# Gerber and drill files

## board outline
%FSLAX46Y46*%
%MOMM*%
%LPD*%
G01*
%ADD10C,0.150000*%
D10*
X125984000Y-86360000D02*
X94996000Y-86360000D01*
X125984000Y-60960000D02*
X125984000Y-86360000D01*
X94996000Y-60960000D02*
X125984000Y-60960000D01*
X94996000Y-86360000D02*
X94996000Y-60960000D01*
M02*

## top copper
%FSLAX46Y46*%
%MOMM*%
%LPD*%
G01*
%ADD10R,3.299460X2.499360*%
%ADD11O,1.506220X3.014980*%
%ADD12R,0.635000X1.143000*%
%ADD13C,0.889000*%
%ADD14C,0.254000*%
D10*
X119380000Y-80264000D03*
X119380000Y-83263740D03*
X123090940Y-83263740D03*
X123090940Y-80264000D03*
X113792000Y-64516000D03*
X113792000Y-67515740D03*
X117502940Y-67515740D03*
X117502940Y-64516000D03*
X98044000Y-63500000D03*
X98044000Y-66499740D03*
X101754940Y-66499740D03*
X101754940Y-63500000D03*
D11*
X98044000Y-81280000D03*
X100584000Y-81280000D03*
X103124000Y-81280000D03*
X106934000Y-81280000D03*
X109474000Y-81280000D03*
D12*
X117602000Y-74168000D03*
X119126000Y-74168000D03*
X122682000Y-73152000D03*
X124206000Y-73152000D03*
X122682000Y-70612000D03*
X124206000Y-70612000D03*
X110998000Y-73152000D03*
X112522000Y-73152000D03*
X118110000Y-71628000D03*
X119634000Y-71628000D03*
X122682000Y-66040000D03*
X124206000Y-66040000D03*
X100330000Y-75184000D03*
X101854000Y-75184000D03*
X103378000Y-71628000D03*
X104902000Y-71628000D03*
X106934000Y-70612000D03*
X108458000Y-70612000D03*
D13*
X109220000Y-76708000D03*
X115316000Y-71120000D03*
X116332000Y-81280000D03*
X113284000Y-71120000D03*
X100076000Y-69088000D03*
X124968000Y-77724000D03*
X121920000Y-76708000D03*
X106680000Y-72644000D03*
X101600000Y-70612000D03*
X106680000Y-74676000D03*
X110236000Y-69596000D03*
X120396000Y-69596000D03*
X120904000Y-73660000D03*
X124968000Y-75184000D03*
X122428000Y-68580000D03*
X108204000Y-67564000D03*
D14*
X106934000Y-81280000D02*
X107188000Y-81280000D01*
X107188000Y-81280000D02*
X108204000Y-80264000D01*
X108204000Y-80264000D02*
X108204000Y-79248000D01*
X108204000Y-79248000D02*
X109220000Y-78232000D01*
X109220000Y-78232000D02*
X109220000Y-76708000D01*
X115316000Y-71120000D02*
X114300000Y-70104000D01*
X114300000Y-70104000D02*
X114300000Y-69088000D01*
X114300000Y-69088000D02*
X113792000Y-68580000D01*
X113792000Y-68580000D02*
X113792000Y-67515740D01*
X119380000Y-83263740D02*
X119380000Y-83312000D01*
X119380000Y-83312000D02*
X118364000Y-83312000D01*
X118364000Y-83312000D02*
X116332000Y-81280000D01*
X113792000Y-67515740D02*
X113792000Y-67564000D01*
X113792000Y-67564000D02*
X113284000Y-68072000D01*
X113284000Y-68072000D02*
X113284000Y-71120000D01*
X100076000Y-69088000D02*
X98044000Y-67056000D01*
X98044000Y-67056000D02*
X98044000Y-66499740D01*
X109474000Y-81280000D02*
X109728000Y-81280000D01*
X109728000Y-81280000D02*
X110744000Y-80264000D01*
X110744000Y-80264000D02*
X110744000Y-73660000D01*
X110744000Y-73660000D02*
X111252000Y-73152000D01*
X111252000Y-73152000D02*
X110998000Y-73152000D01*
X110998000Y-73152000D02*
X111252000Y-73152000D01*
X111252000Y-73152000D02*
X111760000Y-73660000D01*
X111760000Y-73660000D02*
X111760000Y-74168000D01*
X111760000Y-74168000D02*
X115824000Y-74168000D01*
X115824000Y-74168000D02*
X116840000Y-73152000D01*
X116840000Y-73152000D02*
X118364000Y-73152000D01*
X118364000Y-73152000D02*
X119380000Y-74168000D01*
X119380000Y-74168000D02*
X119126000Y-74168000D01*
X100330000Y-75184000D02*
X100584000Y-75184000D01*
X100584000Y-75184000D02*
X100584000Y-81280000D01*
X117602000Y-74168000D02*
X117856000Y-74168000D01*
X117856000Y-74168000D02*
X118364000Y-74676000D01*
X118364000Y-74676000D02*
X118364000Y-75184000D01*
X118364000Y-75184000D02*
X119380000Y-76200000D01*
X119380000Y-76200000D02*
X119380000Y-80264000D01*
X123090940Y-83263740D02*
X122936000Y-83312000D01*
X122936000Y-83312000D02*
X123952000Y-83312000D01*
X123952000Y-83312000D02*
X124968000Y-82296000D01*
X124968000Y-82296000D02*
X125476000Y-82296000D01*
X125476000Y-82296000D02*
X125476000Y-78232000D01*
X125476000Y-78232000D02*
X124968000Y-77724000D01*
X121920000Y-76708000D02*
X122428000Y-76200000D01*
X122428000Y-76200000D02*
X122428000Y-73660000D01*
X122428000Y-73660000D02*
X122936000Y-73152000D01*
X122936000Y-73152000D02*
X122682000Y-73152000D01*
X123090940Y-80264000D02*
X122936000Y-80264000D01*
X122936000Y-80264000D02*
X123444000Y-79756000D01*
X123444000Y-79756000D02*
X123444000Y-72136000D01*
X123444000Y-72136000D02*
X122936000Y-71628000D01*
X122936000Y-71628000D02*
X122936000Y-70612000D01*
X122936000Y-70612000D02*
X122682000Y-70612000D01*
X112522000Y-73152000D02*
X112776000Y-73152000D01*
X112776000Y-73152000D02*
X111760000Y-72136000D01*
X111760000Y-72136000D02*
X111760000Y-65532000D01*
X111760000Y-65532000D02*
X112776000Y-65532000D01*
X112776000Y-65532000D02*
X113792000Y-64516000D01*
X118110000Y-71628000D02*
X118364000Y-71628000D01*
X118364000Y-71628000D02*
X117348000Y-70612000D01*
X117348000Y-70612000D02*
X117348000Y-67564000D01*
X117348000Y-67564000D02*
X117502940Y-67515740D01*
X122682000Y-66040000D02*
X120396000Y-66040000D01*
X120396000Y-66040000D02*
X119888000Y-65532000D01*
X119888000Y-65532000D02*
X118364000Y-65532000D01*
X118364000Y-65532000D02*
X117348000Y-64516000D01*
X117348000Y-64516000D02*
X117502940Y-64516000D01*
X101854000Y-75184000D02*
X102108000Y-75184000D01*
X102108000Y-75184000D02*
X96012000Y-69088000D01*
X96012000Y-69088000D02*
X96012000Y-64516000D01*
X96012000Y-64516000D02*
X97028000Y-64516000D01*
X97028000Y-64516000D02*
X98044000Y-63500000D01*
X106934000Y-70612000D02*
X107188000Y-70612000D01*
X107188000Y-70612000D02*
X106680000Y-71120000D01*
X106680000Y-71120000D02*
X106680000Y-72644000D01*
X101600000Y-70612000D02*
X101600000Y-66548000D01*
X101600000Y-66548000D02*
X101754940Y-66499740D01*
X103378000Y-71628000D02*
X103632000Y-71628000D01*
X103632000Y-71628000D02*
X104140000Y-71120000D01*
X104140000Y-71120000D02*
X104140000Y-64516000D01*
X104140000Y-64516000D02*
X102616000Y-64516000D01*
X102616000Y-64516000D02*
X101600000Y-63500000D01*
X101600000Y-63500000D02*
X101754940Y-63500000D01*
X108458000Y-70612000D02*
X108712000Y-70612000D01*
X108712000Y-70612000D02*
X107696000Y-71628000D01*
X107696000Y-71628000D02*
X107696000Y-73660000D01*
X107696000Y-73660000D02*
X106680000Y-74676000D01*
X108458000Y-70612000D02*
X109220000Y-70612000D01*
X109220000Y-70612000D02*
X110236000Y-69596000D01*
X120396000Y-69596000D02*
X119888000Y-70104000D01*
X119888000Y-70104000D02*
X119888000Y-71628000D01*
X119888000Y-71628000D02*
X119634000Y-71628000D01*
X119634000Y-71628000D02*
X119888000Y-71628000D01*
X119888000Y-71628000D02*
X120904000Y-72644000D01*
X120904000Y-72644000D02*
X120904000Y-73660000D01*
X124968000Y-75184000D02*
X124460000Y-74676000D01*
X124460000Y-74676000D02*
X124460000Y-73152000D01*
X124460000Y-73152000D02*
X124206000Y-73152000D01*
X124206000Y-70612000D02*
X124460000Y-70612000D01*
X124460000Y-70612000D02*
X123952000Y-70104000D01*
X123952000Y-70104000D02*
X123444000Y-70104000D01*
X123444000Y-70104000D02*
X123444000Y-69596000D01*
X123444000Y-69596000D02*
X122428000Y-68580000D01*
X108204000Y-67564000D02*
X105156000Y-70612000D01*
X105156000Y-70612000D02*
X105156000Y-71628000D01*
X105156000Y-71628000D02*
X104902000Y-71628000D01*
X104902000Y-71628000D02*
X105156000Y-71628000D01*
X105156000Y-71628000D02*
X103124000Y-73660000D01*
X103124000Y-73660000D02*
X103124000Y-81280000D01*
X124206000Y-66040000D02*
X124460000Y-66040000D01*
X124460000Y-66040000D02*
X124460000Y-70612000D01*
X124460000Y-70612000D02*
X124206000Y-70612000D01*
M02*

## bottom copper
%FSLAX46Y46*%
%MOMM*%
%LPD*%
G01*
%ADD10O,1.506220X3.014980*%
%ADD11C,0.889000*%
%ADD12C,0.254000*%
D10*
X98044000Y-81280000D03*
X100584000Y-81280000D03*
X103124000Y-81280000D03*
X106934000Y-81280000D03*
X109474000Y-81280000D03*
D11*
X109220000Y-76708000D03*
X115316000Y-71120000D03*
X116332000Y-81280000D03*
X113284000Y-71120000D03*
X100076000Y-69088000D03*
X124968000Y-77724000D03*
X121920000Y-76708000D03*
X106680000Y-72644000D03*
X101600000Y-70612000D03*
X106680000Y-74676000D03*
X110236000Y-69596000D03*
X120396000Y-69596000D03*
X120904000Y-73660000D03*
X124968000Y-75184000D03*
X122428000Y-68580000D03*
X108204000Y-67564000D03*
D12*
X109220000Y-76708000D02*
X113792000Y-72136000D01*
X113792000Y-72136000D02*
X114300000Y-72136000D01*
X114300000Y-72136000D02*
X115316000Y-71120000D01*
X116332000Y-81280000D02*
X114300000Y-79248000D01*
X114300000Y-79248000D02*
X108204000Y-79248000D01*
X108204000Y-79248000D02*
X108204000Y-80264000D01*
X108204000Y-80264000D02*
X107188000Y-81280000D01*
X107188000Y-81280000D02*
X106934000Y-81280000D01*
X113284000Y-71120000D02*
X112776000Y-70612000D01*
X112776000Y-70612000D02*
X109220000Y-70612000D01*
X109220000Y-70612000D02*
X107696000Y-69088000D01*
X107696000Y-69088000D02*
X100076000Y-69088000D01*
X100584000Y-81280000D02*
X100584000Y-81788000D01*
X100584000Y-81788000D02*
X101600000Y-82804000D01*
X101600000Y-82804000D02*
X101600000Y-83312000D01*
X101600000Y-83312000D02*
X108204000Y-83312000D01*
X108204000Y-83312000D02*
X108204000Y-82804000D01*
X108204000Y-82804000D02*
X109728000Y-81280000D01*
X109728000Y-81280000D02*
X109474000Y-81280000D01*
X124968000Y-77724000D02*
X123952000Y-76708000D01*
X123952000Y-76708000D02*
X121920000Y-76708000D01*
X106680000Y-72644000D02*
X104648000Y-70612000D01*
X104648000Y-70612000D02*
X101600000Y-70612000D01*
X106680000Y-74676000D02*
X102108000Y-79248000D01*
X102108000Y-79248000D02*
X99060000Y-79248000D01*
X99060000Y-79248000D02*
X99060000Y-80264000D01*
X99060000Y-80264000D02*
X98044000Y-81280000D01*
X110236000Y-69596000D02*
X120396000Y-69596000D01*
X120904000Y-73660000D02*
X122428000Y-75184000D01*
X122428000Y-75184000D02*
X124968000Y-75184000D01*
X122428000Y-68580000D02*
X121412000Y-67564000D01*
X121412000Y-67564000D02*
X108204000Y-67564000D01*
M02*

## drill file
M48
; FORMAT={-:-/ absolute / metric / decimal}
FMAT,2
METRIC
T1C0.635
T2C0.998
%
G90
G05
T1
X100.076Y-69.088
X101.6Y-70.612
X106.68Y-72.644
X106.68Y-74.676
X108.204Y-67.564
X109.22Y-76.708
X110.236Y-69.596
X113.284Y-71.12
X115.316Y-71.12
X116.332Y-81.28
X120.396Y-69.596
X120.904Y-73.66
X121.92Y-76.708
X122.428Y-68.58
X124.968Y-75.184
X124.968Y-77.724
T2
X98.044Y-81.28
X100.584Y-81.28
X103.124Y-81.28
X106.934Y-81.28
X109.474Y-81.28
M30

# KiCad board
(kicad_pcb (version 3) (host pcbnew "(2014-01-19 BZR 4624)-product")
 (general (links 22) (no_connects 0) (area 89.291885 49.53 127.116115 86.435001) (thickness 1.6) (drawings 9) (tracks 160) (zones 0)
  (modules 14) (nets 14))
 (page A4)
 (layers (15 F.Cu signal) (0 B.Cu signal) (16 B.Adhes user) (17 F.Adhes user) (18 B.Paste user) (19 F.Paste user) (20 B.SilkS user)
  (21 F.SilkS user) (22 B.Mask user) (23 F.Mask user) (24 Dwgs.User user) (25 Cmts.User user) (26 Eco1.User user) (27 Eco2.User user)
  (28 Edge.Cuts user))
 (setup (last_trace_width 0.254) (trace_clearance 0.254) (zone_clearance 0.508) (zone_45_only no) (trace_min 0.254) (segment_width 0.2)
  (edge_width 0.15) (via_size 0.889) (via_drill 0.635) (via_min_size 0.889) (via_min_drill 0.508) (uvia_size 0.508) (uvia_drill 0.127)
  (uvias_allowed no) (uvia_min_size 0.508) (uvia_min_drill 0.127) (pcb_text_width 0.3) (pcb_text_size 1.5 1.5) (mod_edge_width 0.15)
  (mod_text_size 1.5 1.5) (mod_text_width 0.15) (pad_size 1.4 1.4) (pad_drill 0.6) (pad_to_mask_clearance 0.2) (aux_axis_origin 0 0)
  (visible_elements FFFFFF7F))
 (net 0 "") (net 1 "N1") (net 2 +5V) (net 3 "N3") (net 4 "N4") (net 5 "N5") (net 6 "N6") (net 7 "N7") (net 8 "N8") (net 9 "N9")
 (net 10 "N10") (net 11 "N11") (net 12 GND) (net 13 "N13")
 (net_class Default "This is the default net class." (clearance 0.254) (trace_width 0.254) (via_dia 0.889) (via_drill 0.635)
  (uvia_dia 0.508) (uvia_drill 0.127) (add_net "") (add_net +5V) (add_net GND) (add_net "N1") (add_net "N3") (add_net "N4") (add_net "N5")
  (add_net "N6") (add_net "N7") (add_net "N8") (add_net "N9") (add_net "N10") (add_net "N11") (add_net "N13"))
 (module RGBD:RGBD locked (layer F.Cu) (at 119.38 77.724)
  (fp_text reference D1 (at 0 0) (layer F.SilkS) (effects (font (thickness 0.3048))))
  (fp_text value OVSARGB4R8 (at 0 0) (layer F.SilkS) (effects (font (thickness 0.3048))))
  (pad 1 smd rect (at 0 2.54) (size 3.29946 2.49936) (layers F.Cu F.Paste F.Mask) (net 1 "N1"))
  (pad 2 smd rect (at 0 5.53974) (size 3.29946 2.49936) (layers F.Cu F.Paste F.Mask) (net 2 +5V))
  (pad 3 smd rect (at 3.71094 5.53974) (size 3.29946 2.49936) (layers F.Cu F.Paste F.Mask) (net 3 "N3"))
  (pad 4 smd rect (at 3.71094 2.54) (size 3.29946 2.49936) (layers F.Cu F.Paste F.Mask) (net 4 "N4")))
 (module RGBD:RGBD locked (layer F.Cu) (at 113.792 61.976)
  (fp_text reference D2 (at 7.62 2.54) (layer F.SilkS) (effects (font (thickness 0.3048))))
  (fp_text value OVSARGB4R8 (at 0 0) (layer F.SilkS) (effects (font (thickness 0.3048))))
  (pad 1 smd rect (at 0 2.54) (size 3.29946 2.49936) (layers F.Cu F.Paste F.Mask) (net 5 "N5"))
  (pad 2 smd rect (at 0 5.53974) (size 3.29946 2.49936) (layers F.Cu F.Paste F.Mask) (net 2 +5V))
  (pad 3 smd rect (at 3.71094 5.53974) (size 3.29946 2.49936) (layers F.Cu F.Paste F.Mask) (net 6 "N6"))
  (pad 4 smd rect (at 3.71094 2.54) (size 3.29946 2.49936) (layers F.Cu F.Paste F.Mask) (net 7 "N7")))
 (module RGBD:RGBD (layer F.Cu) (at 98.044 60.96)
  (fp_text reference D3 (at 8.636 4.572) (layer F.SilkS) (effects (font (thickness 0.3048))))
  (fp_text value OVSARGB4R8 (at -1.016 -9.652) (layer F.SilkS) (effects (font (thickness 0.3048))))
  (pad 1 smd rect (at 0 2.54) (size 3.29946 2.49936) (layers F.Cu F.Paste F.Mask) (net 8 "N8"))
  (pad 2 smd rect (at 0 5.53974) (size 3.29946 2.49936) (layers F.Cu F.Paste F.Mask) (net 2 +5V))
  (pad 3 smd rect (at 3.71094 5.53974) (size 3.29946 2.49936) (layers F.Cu F.Paste F.Mask) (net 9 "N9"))
  (pad 4 smd rect (at 3.71094 2.54) (size 3.29946 2.49936) (layers F.Cu F.Paste F.Mask) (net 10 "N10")))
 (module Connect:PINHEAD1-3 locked (layer F.Cu) (at 100.584 81.28)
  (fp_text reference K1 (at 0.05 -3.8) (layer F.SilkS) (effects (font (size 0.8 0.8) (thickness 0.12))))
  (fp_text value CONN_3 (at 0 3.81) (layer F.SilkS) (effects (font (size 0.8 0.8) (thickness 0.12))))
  (pad 1 thru_hole oval (at -2.54 0) (size 1.50622 3.01498) (drill 0.99822) (layers *.Cu *.Mask F.SilkS) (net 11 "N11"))
  (pad 2 thru_hole oval (at 0 0) (size 1.50622 3.01498) (drill 0.99822) (layers *.Cu *.Mask F.SilkS) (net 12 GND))
  (pad 3 thru_hole oval (at 2.54 0) (size 1.50622 3.01498) (drill 0.99822) (layers *.Cu *.Mask F.SilkS) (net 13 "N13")))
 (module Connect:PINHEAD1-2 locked (layer F.Cu) (at 108.204 81.28)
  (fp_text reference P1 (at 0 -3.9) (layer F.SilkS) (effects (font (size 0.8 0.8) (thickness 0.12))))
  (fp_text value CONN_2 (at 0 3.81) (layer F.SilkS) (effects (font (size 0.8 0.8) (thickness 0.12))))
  (pad 1 thru_hole oval (at -1.27 0) (size 1.50622 3.01498) (drill 0.99822) (layers *.Cu *.Mask F.SilkS) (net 2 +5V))
  (pad 2 thru_hole oval (at 1.27 0) (size 1.50622 3.01498) (drill 0.99822) (layers *.Cu *.Mask F.SilkS) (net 12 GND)))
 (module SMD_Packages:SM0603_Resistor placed (layer F.Cu) (at 118.364 74.168)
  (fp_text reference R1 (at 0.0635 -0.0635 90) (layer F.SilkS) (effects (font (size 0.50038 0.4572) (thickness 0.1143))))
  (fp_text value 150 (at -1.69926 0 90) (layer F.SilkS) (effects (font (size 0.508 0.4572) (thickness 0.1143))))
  (pad 1 smd rect (at -0.762 0) (size 0.635 1.143) (layers F.Cu F.Paste F.Mask) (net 1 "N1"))
  (pad 2 smd rect (at 0.762 0) (size 0.635 1.143) (layers F.Cu F.Paste F.Mask) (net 12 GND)))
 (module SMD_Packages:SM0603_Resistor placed (layer F.Cu) (at 123.444 73.152)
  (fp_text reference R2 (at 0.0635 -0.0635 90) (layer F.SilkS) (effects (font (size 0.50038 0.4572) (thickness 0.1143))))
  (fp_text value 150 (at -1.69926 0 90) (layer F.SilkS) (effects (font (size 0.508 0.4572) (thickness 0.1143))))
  (pad 1 smd rect (at -0.762 0) (size 0.635 1.143) (layers F.Cu F.Paste F.Mask) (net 3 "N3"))
  (pad 2 smd rect (at 0.762 0) (size 0.635 1.143) (layers F.Cu F.Paste F.Mask) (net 11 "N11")))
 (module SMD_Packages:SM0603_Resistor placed (layer F.Cu) (at 123.444 70.612)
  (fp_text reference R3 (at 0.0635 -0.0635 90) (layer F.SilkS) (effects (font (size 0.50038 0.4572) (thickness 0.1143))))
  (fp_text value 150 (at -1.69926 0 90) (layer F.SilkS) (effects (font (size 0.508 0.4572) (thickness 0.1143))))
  (pad 1 smd rect (at -0.762 0) (size 0.635 1.143) (layers F.Cu F.Paste F.Mask) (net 4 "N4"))
  (pad 2 smd rect (at 0.762 0) (size 0.635 1.143) (layers F.Cu F.Paste F.Mask) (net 13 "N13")))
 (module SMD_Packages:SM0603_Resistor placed (layer F.Cu) (at 111.76 73.152)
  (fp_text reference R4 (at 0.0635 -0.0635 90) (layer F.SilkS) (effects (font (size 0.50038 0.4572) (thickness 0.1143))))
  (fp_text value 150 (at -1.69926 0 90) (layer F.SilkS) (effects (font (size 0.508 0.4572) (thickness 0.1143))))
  (pad 1 smd rect (at -0.762 0) (size 0.635 1.143) (layers F.Cu F.Paste F.Mask) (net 12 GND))
  (pad 2 smd rect (at 0.762 0) (size 0.635 1.143) (layers F.Cu F.Paste F.Mask) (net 5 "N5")))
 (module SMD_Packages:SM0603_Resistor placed (layer F.Cu) (at 118.872 71.628)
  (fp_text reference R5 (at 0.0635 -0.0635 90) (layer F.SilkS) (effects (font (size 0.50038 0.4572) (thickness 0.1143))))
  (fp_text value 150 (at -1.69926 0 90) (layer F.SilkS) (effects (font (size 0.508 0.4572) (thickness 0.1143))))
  (pad 1 smd rect (at -0.762 0) (size 0.635 1.143) (layers F.Cu F.Paste F.Mask) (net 6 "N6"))
  (pad 2 smd rect (at 0.762 0) (size 0.635 1.143) (layers F.Cu F.Paste F.Mask) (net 11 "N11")))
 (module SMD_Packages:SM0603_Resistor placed (layer F.Cu) (at 123.444 66.04)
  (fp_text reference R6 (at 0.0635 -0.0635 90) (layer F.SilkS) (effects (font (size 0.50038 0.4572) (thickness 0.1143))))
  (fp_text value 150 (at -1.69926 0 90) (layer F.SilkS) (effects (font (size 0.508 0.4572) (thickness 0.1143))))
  (pad 1 smd rect (at -0.762 0) (size 0.635 1.143) (layers F.Cu F.Paste F.Mask) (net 7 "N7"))
  (pad 2 smd rect (at 0.762 0) (size 0.635 1.143) (layers F.Cu F.Paste F.Mask) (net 13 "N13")))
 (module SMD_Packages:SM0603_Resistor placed (layer F.Cu) (at 101.092 75.184)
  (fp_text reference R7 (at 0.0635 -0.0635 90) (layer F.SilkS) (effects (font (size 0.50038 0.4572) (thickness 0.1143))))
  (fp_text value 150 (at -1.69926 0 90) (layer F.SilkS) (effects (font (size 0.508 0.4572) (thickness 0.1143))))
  (pad 1 smd rect (at -0.762 0) (size 0.635 1.143) (layers F.Cu F.Paste F.Mask) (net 12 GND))
  (pad 2 smd rect (at 0.762 0) (size 0.635 1.143) (layers F.Cu F.Paste F.Mask) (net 8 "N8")))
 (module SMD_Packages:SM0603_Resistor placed (layer F.Cu) (at 104.14 71.628)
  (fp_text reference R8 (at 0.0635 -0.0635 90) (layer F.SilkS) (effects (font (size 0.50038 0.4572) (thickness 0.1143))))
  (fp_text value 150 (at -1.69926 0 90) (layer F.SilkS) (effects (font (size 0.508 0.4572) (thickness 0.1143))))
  (pad 1 smd rect (at -0.762 0) (size 0.635 1.143) (layers F.Cu F.Paste F.Mask) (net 10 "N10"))
  (pad 2 smd rect (at 0.762 0) (size 0.635 1.143) (layers F.Cu F.Paste F.Mask) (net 13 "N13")))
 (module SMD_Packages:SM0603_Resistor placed (layer F.Cu) (at 107.696 70.612)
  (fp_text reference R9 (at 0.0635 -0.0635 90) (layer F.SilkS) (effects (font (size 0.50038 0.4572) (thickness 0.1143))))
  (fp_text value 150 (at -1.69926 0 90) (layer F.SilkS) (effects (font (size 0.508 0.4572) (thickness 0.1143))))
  (pad 1 smd rect (at -0.762 0) (size 0.635 1.143) (layers F.Cu F.Paste F.Mask) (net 9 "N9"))
  (pad 2 smd rect (at 0.762 0) (size 0.635 1.143) (layers F.Cu F.Paste F.Mask) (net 11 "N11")))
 (gr_line (start 125.984 86.36) (end 94.996 86.36) (angle 90) (layer Edge.Cuts) (width 0.15))
 (gr_line (start 125.984 60.96) (end 125.984 86.36) (angle 90) (layer Edge.Cuts) (width 0.15))
 (gr_line (start 94.996 60.96) (end 125.984 60.96) (angle 90) (layer Edge.Cuts) (width 0.15))
 (gr_line (start 94.996 86.36) (end 94.996 60.96) (angle 90) (layer Edge.Cuts) (width 0.15))
 (segment (start 106.934 81.28) (end 107.188 81.28) (width 0.254) (layer F.Cu) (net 2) (status 80000))
 (segment (start 107.188 81.28) (end 108.204 80.264) (width 0.254) (layer F.Cu) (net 2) (status 80000))
 (segment (start 108.204 80.264) (end 108.204 79.248) (width 0.254) (layer F.Cu) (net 2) (status 80000))
 (segment (start 108.204 79.248) (end 109.22 78.232) (width 0.254) (layer F.Cu) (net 2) (status 80000))
 (segment (start 109.22 78.232) (end 109.22 76.708) (width 0.254) (layer F.Cu) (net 2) (status 80000))
 (via (at 109.22 76.708) (size 0.889) (layers F.Cu B.Cu) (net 2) (status 80000))
 (segment (start 109.22 76.708) (end 113.792 72.136) (width 0.254) (layer B.Cu) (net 2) (status 80000))
 (segment (start 113.792 72.136) (end 114.3 72.136) (width 0.254) (layer B.Cu) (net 2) (status 80000))
 (segment (start 114.3 72.136) (end 115.316 71.12) (width 0.254) (layer B.Cu) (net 2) (status 80000))
 (via (at 115.316 71.12) (size 0.889) (layers F.Cu B.Cu) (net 2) (status 80000))
 (segment (start 115.316 71.12) (end 114.3 70.104) (width 0.254) (layer F.Cu) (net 2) (status 80000))
 (segment (start 114.3 70.104) (end 114.3 69.088) (width 0.254) (layer F.Cu) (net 2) (status 80000))
 (segment (start 114.3 69.088) (end 113.792 68.58) (width 0.254) (layer F.Cu) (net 2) (status 80000))
 (segment (start 113.792 68.58) (end 113.792 67.51574) (width 0.254) (layer F.Cu) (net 2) (status 80000))
 (segment (start 119.38 83.26374) (end 119.38 83.312) (width 0.254) (layer F.Cu) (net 2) (status 80000))
 (segment (start 119.38 83.312) (end 118.364 83.312) (width 0.254) (layer F.Cu) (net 2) (status 80000))
 (segment (start 118.364 83.312) (end 116.332 81.28) (width 0.254) (layer F.Cu) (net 2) (status 80000))
 (via (at 116.332 81.28) (size 0.889) (layers F.Cu B.Cu) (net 2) (status 80000))
 (segment (start 116.332 81.28) (end 114.3 79.248) (width 0.254) (layer B.Cu) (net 2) (status 80000))
 (segment (start 114.3 79.248) (end 108.204 79.248) (width 0.254) (layer B.Cu) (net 2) (status 80000))
 (segment (start 108.204 79.248) (end 108.204 80.264) (width 0.254) (layer B.Cu) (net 2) (status 80000))
 (segment (start 108.204 80.264) (end 107.188 81.28) (width 0.254) (layer B.Cu) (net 2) (status 80000))
 (segment (start 107.188 81.28) (end 106.934 81.28) (width 0.254) (layer B.Cu) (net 2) (status 80000))
 (segment (start 113.792 67.51574) (end 113.792 67.564) (width 0.254) (layer F.Cu) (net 2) (status 80000))
 (segment (start 113.792 67.564) (end 113.284 68.072) (width 0.254) (layer F.Cu) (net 2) (status 80000))
 (segment (start 113.284 68.072) (end 113.284 71.12) (width 0.254) (layer F.Cu) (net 2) (status 80000))
 (via (at 113.284 71.12) (size 0.889) (layers F.Cu B.Cu) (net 2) (status 80000))
 (segment (start 113.284 71.12) (end 112.776 70.612) (width 0.254) (layer B.Cu) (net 2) (status 80000))
 (segment (start 112.776 70.612) (end 109.22 70.612) (width 0.254) (layer B.Cu) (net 2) (status 80000))
 (segment (start 109.22 70.612) (end 107.696 69.088) (width 0.254) (layer B.Cu) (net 2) (status 80000))
 (segment (start 107.696 69.088) (end 100.076 69.088) (width 0.254) (layer B.Cu) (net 2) (status 80000))
 (via (at 100.076 69.088) (size 0.889) (layers F.Cu B.Cu) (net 2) (status 80000))
 (segment (start 100.076 69.088) (end 98.044 67.056) (width 0.254) (layer F.Cu) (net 2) (status 80000))
 (segment (start 98.044 67.056) (end 98.044 66.49974) (width 0.254) (layer F.Cu) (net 2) (status 80000))
 (segment (start 109.474 81.28) (end 109.728 81.28) (width 0.254) (layer F.Cu) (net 12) (status 80000))
 (segment (start 109.728 81.28) (end 110.744 80.264) (width 0.254) (layer F.Cu) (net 12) (status 80000))
 (segment (start 110.744 80.264) (end 110.744 73.66) (width 0.254) (layer F.Cu) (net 12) (status 80000))
 (segment (start 110.744 73.66) (end 111.252 73.152) (width 0.254) (layer F.Cu) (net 12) (status 80000))
 (segment (start 111.252 73.152) (end 110.998 73.152) (width 0.254) (layer F.Cu) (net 12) (status 80000))
 (segment (start 110.998 73.152) (end 111.252 73.152) (width 0.254) (layer F.Cu) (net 12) (status 80000))
 (segment (start 111.252 73.152) (end 111.76 73.66) (width 0.254) (layer F.Cu) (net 12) (status 80000))
 (segment (start 111.76 73.66) (end 111.76 74.168) (width 0.254) (layer F.Cu) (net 12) (status 80000))
 (segment (start 111.76 74.168) (end 115.824 74.168) (width 0.254) (layer F.Cu) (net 12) (status 80000))
 (segment (start 115.824 74.168) (end 116.84 73.152) (width 0.254) (layer F.Cu) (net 12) (status 80000))
 (segment (start 116.84 73.152) (end 118.364 73.152) (width 0.254) (layer F.Cu) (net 12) (status 80000))
 (segment (start 118.364 73.152) (end 119.38 74.168) (width 0.254) (layer F.Cu) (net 12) (status 80000))
 (segment (start 119.38 74.168) (end 119.126 74.168) (width 0.254) (layer F.Cu) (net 12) (status 80000))
 (segment (start 100.584 81.28) (end 100.584 81.788) (width 0.254) (layer B.Cu) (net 12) (status 80000))
 (segment (start 100.584 81.788) (end 101.6 82.804) (width 0.254) (layer B.Cu) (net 12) (status 80000))
 (segment (start 101.6 82.804) (end 101.6 83.312) (width 0.254) (layer B.Cu) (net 12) (status 80000))
 (segment (start 101.6 83.312) (end 108.204 83.312) (width 0.254) (layer B.Cu) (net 12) (status 80000))
 (segment (start 108.204 83.312) (end 108.204 82.804) (width 0.254) (layer B.Cu) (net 12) (status 80000))
 (segment (start 108.204 82.804) (end 109.728 81.28) (width 0.254) (layer B.Cu) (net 12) (status 80000))
 (segment (start 109.728 81.28) (end 109.474 81.28) (width 0.254) (layer B.Cu) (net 12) (status 80000))
 (segment (start 100.33 75.184) (end 100.584 75.184) (width 0.254) (layer F.Cu) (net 12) (status 80000))
 (segment (start 100.584 75.184) (end 100.584 81.28) (width 0.254) (layer F.Cu) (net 12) (status 80000))
 (segment (start 117.602 74.168) (end 117.856 74.168) (width 0.254) (layer F.Cu) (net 1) (status 80000))
 (segment (start 117.856 74.168) (end 118.364 74.676) (width 0.254) (layer F.Cu) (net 1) (status 80000))
 (segment (start 118.364 74.676) (end 118.364 75.184) (width 0.254) (layer F.Cu) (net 1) (status 80000))
 (segment (start 118.364 75.184) (end 119.38 76.2) (width 0.254) (layer F.Cu) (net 1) (status 80000))
 (segment (start 119.38 76.2) (end 119.38 80.264) (width 0.254) (layer F.Cu) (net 1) (status 80000))
 (segment (start 123.09094 83.26374) (end 122.936 83.312) (width 0.254) (layer F.Cu) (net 3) (status 80000))
 (segment (start 122.936 83.312) (end 123.952 83.312) (width 0.254) (layer F.Cu) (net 3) (status 80000))
 (segment (start 123.952 83.312) (end 124.968 82.296) (width 0.254) (layer F.Cu) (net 3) (status 80000))
 (segment (start 124.968 82.296) (end 125.476 82.296) (width 0.254) (layer F.Cu) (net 3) (status 80000))
 (segment (start 125.476 82.296) (end 125.476 78.232) (width 0.254) (layer F.Cu) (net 3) (status 80000))
 (segment (start 125.476 78.232) (end 124.968 77.724) (width 0.254) (layer F.Cu) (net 3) (status 80000))
 (via (at 124.968 77.724) (size 0.889) (layers F.Cu B.Cu) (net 3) (status 80000))
 (segment (start 124.968 77.724) (end 123.952 76.708) (width 0.254) (layer B.Cu) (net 3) (status 80000))
 (segment (start 123.952 76.708) (end 121.92 76.708) (width 0.254) (layer B.Cu) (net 3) (status 80000))
 (via (at 121.92 76.708) (size 0.889) (layers F.Cu B.Cu) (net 3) (status 80000))
 (segment (start 121.92 76.708) (end 122.428 76.2) (width 0.254) (layer F.Cu) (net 3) (status 80000))
 (segment (start 122.428 76.2) (end 122.428 73.66) (width 0.254) (layer F.Cu) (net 3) (status 80000))
 (segment (start 122.428 73.66) (end 122.936 73.152) (width 0.254) (layer F.Cu) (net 3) (status 80000))
 (segment (start 122.936 73.152) (end 122.682 73.152) (width 0.254) (layer F.Cu) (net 3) (status 80000))
 (segment (start 123.09094 80.264) (end 122.936 80.264) (width 0.254) (layer F.Cu) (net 4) (status 80000))
 (segment (start 122.936 80.264) (end 123.444 79.756) (width 0.254) (layer F.Cu) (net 4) (status 80000))
 (segment (start 123.444 79.756) (end 123.444 72.136) (width 0.254) (layer F.Cu) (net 4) (status 80000))
 (segment (start 123.444 72.136) (end 122.936 71.628) (width 0.254) (layer F.Cu) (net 4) (status 80000))
 (segment (start 122.936 71.628) (end 122.936 70.612) (width 0.254) (layer F.Cu) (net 4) (status 80000))
 (segment (start 122.936 70.612) (end 122.682 70.612) (width 0.254) (layer F.Cu) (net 4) (status 80000))
 (segment (start 112.522 73.152) (end 112.776 73.152) (width 0.254) (layer F.Cu) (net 5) (status 80000))
 (segment (start 112.776 73.152) (end 111.76 72.136) (width 0.254) (layer F.Cu) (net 5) (status 80000))
 (segment (start 111.76 72.136) (end 111.76 65.532) (width 0.254) (layer F.Cu) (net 5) (status 80000))
 (segment (start 111.76 65.532) (end 112.776 65.532) (width 0.254) (layer F.Cu) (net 5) (status 80000))
 (segment (start 112.776 65.532) (end 113.792 64.516) (width 0.254) (layer F.Cu) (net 5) (status 80000))
 (segment (start 118.11 71.628) (end 118.364 71.628) (width 0.254) (layer F.Cu) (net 6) (status 80000))
 (segment (start 118.364 71.628) (end 117.348 70.612) (width 0.254) (layer F.Cu) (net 6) (status 80000))
 (segment (start 117.348 70.612) (end 117.348 67.564) (width 0.254) (layer F.Cu) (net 6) (status 80000))
 (segment (start 117.348 67.564) (end 117.50294 67.51574) (width 0.254) (layer F.Cu) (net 6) (status 80000))
 (segment (start 122.682 66.04) (end 120.396 66.04) (width 0.254) (layer F.Cu) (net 7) (status 80000))
 (segment (start 120.396 66.04) (end 119.888 65.532) (width 0.254) (layer F.Cu) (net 7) (status 80000))
 (segment (start 119.888 65.532) (end 118.364 65.532) (width 0.254) (layer F.Cu) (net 7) (status 80000))
 (segment (start 118.364 65.532) (end 117.348 64.516) (width 0.254) (layer F.Cu) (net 7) (status 80000))
 (segment (start 117.348 64.516) (end 117.50294 64.516) (width 0.254) (layer F.Cu) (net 7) (status 80000))
 (segment (start 101.854 75.184) (end 102.108 75.184) (width 0.254) (layer F.Cu) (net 8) (status 80000))
 (segment (start 102.108 75.184) (end 96.012 69.088) (width 0.254) (layer F.Cu) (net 8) (status 80000))
 (segment (start 96.012 69.088) (end 96.012 64.516) (width 0.254) (layer F.Cu) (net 8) (status 80000))
 (segment (start 96.012 64.516) (end 97.028 64.516) (width 0.254) (layer F.Cu) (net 8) (status 80000))
 (segment (start 97.028 64.516) (end 98.044 63.5) (width 0.254) (layer F.Cu) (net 8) (status 80000))
 (segment (start 106.934 70.612) (end 107.188 70.612) (width 0.254) (layer F.Cu) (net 9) (status 80000))
 (segment (start 107.188 70.612) (end 106.68 71.12) (width 0.254) (layer F.Cu) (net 9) (status 80000))
 (segment (start 106.68 71.12) (end 106.68 72.644) (width 0.254) (layer F.Cu) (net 9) (status 80000))
 (via (at 106.68 72.644) (size 0.889) (layers F.Cu B.Cu) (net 9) (status 80000))
 (segment (start 106.68 72.644) (end 104.648 70.612) (width 0.254) (layer B.Cu) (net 9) (status 80000))
 (segment (start 104.648 70.612) (end 101.6 70.612) (width 0.254) (layer B.Cu) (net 9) (status 80000))
 (via (at 101.6 70.612) (size 0.889) (layers F.Cu B.Cu) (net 9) (status 80000))
 (segment (start 101.6 70.612) (end 101.6 66.548) (width 0.254) (layer F.Cu) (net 9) (status 80000))
 (segment (start 101.6 66.548) (end 101.75494 66.49974) (width 0.254) (layer F.Cu) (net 9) (status 80000))
 (segment (start 103.378 71.628) (end 103.632 71.628) (width 0.254) (layer F.Cu) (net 10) (status 80000))
 (segment (start 103.632 71.628) (end 104.14 71.12) (width 0.254) (layer F.Cu) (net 10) (status 80000))
 (segment (start 104.14 71.12) (end 104.14 64.516) (width 0.254) (layer F.Cu) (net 10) (status 80000))
 (segment (start 104.14 64.516) (end 102.616 64.516) (width 0.254) (layer F.Cu) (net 10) (status 80000))
 (segment (start 102.616 64.516) (end 101.6 63.5) (width 0.254) (layer F.Cu) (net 10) (status 80000))
 (segment (start 101.6 63.5) (end 101.75494 63.5) (width 0.254) (layer F.Cu) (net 10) (status 80000))
 (segment (start 108.458 70.612) (end 108.712 70.612) (width 0.254) (layer F.Cu) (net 11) (status 80000))
 (segment (start 108.712 70.612) (end 107.696 71.628) (width 0.254) (layer F.Cu) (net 11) (status 80000))
 (segment (start 107.696 71.628) (end 107.696 73.66) (width 0.254) (layer F.Cu) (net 11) (status 80000))
 (segment (start 107.696 73.66) (end 106.68 74.676) (width 0.254) (layer F.Cu) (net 11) (status 80000))
 (via (at 106.68 74.676) (size 0.889) (layers F.Cu B.Cu) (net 11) (status 80000))
 (segment (start 106.68 74.676) (end 102.108 79.248) (width 0.254) (layer B.Cu) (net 11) (status 80000))
 (segment (start 102.108 79.248) (end 99.06 79.248) (width 0.254) (layer B.Cu) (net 11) (status 80000))
 (segment (start 99.06 79.248) (end 99.06 80.264) (width 0.254) (layer B.Cu) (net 11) (status 80000))
 (segment (start 99.06 80.264) (end 98.044 81.28) (width 0.254) (layer B.Cu) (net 11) (status 80000))
 (segment (start 108.458 70.612) (end 109.22 70.612) (width 0.254) (layer F.Cu) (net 11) (status 80000))
 (segment (start 109.22 70.612) (end 110.236 69.596) (width 0.254) (layer F.Cu) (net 11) (status 80000))
 (via (at 110.236 69.596) (size 0.889) (layers F.Cu B.Cu) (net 11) (status 80000))
 (segment (start 110.236 69.596) (end 120.396 69.596) (width 0.254) (layer B.Cu) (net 11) (status 80000))
 (via (at 120.396 69.596) (size 0.889) (layers F.Cu B.Cu) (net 11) (status 80000))
 (segment (start 120.396 69.596) (end 119.888 70.104) (width 0.254) (layer F.Cu) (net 11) (status 80000))
 (segment (start 119.888 70.104) (end 119.888 71.628) (width 0.254) (layer F.Cu) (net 11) (status 80000))
 (segment (start 119.888 71.628) (end 119.634 71.628) (width 0.254) (layer F.Cu) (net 11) (status 80000))
 (segment (start 119.634 71.628) (end 119.888 71.628) (width 0.254) (layer F.Cu) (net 11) (status 80000))
 (segment (start 119.888 71.628) (end 120.904 72.644) (width 0.254) (layer F.Cu) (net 11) (status 80000))
 (segment (start 120.904 72.644) (end 120.904 73.66) (width 0.254) (layer F.Cu) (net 11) (status 80000))
 (via (at 120.904 73.66) (size 0.889) (layers F.Cu B.Cu) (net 11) (status 80000))
 (segment (start 120.904 73.66) (end 122.428 75.184) (width 0.254) (layer B.Cu) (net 11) (status 80000))
 (segment (start 122.428 75.184) (end 124.968 75.184) (width 0.254) (layer B.Cu) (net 11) (status 80000))
 (via (at 124.968 75.184) (size 0.889) (layers F.Cu B.Cu) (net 11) (status 80000))
 (segment (start 124.968 75.184) (end 124.46 74.676) (width 0.254) (layer F.Cu) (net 11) (status 80000))
 (segment (start 124.46 74.676) (end 124.46 73.152) (width 0.254) (layer F.Cu) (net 11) (status 80000))
 (segment (start 124.46 73.152) (end 124.206 73.152) (width 0.254) (layer F.Cu) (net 11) (status 80000))
 (segment (start 124.206 70.612) (end 124.46 70.612) (width 0.254) (layer F.Cu) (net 13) (status 80000))
 (segment (start 124.46 70.612) (end 123.952 70.104) (width 0.254) (layer F.Cu) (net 13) (status 80000))
 (segment (start 123.952 70.104) (end 123.444 70.104) (width 0.254) (layer F.Cu) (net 13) (status 80000))
 (segment (start 123.444 70.104) (end 123.444 69.596) (width 0.254) (layer F.Cu) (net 13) (status 80000))
 (segment (start 123.444 69.596) (end 122.428 68.58) (width 0.254) (layer F.Cu) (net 13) (status 80000))
 (via (at 122.428 68.58) (size 0.889) (layers F.Cu B.Cu) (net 13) (status 80000))
 (segment (start 122.428 68.58) (end 121.412 67.564) (width 0.254) (layer B.Cu) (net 13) (status 80000))
 (segment (start 121.412 67.564) (end 108.204 67.564) (width 0.254) (layer B.Cu) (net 13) (status 80000))
 (via (at 108.204 67.564) (size 0.889) (layers F.Cu B.Cu) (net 13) (status 80000))
 (segment (start 108.204 67.564) (end 105.156 70.612) (width 0.254) (layer F.Cu) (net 13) (status 80000))
 (segment (start 105.156 70.612) (end 105.156 71.628) (width 0.254) (layer F.Cu) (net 13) (status 80000))
 (segment (start 105.156 71.628) (end 104.902 71.628) (width 0.254) (layer F.Cu) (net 13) (status 80000))
 (segment (start 104.902 71.628) (end 105.156 71.628) (width 0.254) (layer F.Cu) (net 13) (status 80000))
 (segment (start 105.156 71.628) (end 103.124 73.66) (width 0.254) (layer F.Cu) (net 13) (status 80000))
 (segment (start 103.124 73.66) (end 103.124 81.28) (width 0.254) (layer F.Cu) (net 13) (status 80000))
 (segment (start 124.206 66.04) (end 124.46 66.04) (width 0.254) (layer F.Cu) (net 13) (status 80000))
 (segment (start 124.46 66.04) (end 124.46 70.612) (width 0.254) (layer F.Cu) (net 13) (status 80000))
 (segment (start 124.46 70.612) (end 124.206 70.612) (width 0.254) (layer F.Cu) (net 13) (status 80000)))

